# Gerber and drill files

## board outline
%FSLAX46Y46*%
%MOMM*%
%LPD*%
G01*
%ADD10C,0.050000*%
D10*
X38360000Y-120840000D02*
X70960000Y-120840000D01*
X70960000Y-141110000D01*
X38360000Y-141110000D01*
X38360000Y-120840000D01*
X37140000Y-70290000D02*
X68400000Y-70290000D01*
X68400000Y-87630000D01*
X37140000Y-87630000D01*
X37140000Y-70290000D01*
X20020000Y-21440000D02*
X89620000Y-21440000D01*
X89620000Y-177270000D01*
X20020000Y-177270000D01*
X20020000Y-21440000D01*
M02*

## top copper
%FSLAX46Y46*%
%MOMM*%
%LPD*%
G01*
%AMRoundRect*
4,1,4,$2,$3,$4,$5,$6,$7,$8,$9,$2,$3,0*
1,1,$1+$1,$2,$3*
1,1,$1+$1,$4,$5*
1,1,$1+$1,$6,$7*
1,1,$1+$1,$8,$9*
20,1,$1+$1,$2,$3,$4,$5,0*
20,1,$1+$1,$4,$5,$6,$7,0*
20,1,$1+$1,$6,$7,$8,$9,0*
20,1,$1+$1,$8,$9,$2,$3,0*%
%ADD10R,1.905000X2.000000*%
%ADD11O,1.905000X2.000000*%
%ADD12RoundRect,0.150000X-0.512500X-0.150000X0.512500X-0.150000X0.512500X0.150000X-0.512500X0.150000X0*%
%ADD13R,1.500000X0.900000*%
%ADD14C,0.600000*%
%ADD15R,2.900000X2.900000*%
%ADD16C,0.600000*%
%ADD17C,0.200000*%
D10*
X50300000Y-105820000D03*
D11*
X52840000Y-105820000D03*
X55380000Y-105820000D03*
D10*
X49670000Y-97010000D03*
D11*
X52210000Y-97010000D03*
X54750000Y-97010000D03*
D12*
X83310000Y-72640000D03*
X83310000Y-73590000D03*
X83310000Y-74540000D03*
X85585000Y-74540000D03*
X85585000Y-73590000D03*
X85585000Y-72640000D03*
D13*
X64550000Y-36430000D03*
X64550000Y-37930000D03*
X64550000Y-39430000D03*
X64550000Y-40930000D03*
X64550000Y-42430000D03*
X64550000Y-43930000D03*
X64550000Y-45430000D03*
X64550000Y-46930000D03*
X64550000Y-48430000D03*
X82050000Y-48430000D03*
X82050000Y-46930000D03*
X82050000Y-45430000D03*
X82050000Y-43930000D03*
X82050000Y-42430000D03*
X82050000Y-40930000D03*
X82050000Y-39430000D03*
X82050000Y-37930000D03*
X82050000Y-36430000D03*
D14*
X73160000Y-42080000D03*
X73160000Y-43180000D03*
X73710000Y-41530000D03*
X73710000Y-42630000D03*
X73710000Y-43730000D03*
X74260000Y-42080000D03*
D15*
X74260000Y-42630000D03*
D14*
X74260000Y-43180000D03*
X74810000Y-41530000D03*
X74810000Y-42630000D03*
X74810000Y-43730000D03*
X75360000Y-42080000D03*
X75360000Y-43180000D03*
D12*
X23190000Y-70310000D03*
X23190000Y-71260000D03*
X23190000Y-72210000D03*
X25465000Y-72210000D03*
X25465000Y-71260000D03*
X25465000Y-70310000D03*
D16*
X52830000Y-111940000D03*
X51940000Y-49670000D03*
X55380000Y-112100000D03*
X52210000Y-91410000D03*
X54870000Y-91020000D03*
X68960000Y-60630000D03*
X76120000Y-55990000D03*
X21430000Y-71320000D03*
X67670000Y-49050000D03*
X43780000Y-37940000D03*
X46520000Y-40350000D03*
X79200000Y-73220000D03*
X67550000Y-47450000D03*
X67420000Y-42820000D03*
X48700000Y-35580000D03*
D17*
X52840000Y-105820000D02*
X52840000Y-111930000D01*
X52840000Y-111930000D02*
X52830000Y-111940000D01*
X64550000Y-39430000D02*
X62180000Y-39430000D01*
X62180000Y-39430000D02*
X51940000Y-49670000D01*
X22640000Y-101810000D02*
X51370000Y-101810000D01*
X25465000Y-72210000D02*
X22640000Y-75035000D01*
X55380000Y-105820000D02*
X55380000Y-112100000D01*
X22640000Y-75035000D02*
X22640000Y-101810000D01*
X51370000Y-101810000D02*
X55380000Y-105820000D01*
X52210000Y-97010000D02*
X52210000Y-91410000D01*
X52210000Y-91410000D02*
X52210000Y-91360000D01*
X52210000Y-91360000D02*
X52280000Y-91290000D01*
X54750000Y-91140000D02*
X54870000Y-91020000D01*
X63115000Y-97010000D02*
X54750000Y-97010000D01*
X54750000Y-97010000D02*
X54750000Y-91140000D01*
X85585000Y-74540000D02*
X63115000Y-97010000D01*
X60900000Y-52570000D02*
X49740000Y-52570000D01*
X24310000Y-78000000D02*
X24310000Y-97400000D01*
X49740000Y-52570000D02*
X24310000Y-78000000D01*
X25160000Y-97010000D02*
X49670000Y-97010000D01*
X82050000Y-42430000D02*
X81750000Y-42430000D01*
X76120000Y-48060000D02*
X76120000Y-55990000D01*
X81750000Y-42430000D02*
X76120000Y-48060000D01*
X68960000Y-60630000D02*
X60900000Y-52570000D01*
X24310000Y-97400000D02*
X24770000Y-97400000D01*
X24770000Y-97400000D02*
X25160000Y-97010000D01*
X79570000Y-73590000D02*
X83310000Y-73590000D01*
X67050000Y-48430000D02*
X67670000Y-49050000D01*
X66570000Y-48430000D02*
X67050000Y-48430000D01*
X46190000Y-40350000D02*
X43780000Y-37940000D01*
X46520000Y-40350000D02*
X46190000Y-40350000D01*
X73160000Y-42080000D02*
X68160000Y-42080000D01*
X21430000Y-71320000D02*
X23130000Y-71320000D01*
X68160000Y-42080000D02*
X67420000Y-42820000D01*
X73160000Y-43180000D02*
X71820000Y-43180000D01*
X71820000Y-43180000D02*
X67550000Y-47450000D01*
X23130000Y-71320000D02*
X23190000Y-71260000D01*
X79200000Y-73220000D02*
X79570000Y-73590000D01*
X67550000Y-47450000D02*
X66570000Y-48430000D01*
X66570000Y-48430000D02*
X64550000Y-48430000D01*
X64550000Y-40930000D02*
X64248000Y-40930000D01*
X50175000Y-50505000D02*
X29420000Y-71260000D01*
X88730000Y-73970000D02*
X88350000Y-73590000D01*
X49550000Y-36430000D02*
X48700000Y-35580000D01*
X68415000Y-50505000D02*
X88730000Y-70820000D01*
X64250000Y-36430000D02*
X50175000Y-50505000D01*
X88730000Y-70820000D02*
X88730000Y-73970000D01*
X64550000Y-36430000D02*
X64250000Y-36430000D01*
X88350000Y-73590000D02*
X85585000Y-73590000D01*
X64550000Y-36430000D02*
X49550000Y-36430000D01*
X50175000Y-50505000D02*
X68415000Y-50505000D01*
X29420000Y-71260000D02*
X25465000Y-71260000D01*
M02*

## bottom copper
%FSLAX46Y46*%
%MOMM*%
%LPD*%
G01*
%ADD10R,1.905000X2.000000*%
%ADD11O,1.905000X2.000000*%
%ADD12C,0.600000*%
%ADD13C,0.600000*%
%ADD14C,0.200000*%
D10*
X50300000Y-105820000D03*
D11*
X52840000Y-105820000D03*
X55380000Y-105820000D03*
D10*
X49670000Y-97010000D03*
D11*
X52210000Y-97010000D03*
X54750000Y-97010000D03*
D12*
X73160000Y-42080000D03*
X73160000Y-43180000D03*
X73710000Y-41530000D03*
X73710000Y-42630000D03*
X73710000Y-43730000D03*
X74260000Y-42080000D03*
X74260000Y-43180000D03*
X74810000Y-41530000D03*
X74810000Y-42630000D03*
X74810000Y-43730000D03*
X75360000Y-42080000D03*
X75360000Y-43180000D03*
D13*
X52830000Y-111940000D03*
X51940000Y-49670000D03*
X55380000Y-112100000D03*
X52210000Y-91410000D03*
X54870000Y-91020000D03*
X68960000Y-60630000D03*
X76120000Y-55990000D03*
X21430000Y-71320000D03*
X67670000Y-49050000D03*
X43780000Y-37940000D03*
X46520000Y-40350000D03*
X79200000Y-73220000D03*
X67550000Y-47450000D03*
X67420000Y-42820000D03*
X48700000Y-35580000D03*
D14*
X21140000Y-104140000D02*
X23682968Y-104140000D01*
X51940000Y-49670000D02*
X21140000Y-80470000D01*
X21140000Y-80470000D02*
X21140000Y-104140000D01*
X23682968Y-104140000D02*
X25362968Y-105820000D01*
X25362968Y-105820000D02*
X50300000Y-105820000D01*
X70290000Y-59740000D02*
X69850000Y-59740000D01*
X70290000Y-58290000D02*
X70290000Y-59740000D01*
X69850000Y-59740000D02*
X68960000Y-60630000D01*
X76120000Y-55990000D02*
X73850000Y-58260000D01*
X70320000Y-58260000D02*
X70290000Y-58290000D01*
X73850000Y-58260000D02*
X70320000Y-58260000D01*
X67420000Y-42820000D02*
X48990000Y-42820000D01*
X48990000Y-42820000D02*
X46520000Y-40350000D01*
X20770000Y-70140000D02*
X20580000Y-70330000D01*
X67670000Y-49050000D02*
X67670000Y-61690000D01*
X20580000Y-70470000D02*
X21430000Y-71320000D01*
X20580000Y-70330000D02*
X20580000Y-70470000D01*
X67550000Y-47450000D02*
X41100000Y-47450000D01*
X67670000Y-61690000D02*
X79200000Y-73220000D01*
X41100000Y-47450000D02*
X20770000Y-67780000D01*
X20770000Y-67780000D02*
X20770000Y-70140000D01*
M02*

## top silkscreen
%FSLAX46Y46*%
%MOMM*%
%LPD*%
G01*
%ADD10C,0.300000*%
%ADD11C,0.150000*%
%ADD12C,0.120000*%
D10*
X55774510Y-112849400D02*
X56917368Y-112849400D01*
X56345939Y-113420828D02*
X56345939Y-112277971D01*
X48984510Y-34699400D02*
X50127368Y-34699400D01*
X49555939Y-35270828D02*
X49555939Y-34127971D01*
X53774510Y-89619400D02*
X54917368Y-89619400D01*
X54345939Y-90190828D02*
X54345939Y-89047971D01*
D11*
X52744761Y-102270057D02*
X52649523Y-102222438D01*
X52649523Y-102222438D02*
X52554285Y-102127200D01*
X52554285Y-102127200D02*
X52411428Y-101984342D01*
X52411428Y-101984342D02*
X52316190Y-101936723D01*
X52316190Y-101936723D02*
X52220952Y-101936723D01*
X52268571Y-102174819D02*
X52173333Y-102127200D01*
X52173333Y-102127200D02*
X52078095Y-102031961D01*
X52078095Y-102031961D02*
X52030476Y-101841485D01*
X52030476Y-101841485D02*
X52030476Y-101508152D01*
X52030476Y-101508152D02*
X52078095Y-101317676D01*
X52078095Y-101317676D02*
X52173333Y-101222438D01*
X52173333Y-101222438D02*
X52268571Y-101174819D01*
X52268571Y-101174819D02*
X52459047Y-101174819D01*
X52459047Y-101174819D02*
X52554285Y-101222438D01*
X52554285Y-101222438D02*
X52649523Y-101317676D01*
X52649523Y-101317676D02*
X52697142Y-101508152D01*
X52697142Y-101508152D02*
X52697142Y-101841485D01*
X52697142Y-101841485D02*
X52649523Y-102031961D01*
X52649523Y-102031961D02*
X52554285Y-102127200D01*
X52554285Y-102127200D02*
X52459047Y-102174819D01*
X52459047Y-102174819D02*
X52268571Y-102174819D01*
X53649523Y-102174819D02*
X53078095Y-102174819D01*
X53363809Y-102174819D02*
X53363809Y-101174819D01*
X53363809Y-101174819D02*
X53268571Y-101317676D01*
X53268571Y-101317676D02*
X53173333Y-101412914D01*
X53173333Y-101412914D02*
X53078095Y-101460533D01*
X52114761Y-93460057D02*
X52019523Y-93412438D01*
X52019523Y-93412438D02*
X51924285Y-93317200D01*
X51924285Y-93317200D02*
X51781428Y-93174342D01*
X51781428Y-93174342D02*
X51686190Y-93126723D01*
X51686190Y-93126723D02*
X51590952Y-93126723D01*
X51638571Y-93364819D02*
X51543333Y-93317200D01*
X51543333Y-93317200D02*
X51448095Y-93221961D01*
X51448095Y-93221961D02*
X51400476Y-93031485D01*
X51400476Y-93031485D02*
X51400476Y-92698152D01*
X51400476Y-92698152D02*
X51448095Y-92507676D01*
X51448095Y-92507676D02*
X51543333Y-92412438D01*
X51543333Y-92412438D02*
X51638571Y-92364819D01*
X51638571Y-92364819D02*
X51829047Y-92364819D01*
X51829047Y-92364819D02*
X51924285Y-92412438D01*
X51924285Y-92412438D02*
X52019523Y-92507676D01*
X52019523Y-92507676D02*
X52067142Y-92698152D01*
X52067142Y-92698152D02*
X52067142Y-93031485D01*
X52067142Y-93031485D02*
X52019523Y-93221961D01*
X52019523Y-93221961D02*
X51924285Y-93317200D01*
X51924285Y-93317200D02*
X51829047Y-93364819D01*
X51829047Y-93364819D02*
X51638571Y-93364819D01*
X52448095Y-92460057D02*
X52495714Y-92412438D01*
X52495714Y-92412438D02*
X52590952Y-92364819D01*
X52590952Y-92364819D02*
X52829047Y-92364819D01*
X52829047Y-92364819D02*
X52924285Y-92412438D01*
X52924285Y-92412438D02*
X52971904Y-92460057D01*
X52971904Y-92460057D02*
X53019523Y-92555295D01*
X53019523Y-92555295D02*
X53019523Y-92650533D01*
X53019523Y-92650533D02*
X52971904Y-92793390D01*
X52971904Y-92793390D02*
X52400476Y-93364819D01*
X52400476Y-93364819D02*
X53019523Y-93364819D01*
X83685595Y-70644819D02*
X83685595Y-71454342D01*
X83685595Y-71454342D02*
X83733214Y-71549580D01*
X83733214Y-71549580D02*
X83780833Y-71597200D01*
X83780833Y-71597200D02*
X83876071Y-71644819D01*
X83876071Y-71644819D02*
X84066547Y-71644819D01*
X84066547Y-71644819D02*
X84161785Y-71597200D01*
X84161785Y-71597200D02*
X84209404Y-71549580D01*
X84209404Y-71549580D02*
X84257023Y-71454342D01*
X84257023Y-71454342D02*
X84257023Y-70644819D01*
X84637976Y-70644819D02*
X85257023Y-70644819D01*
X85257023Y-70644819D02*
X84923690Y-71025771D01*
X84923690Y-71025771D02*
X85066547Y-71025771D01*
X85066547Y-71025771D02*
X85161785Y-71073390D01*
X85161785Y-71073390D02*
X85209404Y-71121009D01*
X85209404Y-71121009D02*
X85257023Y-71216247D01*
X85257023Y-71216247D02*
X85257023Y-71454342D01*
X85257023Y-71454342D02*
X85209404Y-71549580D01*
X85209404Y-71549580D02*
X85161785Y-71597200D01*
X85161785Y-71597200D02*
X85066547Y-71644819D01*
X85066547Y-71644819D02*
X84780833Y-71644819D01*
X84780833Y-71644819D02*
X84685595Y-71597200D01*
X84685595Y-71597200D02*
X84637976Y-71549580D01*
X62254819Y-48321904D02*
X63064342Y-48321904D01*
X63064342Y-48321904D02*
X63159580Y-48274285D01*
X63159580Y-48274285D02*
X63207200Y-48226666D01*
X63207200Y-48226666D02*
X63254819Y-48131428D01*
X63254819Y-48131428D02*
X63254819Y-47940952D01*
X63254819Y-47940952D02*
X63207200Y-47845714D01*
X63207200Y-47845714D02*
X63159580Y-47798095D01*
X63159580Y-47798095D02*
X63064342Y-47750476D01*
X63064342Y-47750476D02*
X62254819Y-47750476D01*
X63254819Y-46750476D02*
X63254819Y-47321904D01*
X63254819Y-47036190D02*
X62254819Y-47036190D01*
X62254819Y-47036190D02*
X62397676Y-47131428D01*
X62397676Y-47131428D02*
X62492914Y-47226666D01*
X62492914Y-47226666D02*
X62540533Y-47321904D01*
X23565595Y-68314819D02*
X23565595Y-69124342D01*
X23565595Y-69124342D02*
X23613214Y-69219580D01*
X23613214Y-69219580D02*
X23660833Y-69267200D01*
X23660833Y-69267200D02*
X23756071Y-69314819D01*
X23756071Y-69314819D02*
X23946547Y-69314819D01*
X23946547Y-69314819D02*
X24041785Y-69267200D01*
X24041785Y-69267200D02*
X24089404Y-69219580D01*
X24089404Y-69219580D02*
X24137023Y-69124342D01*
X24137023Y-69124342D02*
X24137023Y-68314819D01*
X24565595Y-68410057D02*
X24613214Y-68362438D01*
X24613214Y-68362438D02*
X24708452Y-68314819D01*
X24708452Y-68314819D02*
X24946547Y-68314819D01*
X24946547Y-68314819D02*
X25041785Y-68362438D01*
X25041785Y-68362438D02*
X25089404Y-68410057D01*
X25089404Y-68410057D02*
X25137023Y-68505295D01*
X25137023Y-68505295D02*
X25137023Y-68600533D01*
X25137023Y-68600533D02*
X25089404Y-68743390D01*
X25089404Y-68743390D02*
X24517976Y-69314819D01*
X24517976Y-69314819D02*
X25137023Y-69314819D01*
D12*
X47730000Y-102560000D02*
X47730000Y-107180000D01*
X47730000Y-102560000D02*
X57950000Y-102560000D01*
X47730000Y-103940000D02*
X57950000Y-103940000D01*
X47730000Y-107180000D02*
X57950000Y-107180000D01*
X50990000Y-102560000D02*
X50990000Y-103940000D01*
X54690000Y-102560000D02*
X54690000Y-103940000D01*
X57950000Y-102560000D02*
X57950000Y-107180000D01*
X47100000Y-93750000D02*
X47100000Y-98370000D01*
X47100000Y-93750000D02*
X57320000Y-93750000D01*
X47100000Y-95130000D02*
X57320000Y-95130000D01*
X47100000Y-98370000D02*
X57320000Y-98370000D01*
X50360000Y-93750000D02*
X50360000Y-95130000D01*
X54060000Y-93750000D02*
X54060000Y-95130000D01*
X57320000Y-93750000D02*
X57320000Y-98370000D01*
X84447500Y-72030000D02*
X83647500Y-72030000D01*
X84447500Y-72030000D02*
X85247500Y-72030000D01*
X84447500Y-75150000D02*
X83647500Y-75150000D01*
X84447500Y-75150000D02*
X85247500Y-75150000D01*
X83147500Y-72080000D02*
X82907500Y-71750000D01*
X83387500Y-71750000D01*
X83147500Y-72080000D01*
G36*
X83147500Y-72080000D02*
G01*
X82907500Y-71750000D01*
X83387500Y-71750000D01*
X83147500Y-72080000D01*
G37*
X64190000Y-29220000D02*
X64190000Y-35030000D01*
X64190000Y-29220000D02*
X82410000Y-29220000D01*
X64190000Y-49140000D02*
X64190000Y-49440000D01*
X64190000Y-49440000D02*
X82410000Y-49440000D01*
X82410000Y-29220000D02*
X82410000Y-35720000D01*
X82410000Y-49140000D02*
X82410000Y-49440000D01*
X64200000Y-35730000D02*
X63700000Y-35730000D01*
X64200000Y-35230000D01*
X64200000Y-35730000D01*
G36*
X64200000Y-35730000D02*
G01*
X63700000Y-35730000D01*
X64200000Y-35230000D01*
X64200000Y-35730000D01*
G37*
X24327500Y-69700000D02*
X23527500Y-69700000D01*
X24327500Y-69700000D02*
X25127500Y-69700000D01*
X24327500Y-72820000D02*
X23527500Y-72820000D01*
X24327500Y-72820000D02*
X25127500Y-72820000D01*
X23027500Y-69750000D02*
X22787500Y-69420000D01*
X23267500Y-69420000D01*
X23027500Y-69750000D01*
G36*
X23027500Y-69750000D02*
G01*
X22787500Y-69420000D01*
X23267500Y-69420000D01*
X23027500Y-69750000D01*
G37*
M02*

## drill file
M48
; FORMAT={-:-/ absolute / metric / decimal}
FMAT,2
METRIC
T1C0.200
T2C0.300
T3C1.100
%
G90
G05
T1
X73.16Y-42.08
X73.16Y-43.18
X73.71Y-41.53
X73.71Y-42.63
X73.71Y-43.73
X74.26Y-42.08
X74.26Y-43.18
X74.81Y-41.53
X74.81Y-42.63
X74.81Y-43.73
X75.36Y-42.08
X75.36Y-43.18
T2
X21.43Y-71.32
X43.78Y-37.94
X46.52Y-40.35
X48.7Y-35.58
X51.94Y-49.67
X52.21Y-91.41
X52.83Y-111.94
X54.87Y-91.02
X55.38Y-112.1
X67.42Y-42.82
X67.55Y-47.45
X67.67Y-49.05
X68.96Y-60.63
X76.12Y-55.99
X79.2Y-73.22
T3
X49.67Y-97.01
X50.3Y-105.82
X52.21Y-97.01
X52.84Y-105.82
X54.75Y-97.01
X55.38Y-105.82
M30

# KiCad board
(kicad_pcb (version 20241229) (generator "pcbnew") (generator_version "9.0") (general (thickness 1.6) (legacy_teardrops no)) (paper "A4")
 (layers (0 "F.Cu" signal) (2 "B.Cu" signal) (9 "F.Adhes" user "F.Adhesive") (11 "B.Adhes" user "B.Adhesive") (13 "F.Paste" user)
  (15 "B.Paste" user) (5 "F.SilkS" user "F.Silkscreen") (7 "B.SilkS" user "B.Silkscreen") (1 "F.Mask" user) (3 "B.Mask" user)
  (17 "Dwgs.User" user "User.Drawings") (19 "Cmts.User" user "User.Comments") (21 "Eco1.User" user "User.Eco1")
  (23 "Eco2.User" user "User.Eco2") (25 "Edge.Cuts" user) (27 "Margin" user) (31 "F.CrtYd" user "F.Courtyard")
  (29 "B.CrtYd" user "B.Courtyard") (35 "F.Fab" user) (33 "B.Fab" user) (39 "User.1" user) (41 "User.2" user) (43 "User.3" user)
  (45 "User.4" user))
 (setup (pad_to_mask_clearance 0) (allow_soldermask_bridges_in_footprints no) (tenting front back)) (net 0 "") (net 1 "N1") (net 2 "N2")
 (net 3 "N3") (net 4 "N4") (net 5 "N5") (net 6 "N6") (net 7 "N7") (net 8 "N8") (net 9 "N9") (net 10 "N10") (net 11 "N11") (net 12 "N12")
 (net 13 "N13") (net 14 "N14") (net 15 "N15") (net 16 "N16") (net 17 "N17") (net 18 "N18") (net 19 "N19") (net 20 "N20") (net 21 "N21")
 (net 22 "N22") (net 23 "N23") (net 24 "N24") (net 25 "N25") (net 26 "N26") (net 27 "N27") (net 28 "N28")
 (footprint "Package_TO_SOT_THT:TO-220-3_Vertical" (layer "F.Cu") (at 50.3 105.82)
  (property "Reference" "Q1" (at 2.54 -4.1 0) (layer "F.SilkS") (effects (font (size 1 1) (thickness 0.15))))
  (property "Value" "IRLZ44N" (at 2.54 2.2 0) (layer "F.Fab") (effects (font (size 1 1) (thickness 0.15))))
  (fp_line (start -2.57 -3.26) (end -2.57 1.36) (stroke (width 0.12) (type solid)) (layer "F.SilkS"))
  (fp_line (start -2.57 -3.26) (end 7.65 -3.26) (stroke (width 0.12) (type solid)) (layer "F.SilkS"))
  (fp_line (start -2.57 -1.88) (end 7.65 -1.88) (stroke (width 0.12) (type solid)) (layer "F.SilkS"))
  (fp_line (start -2.57 1.36) (end 7.65 1.36) (stroke (width 0.12) (type solid)) (layer "F.SilkS"))
  (fp_line (start 0.69 -3.26) (end 0.69 -1.88) (stroke (width 0.12) (type solid)) (layer "F.SilkS"))
  (fp_line (start 4.39 -3.26) (end 4.39 -1.88) (stroke (width 0.12) (type solid)) (layer "F.SilkS"))
  (fp_line (start 7.65 -3.26) (end 7.65 1.36) (stroke (width 0.12) (type solid)) (layer "F.SilkS"))
  (pad "1" thru_hole rect (at 0 0) (size 1.905 2) (drill 1.1) (layers "*.Cu" "*.Mask") (remove_unused_layers no) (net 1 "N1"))
  (pad "2" thru_hole oval (at 2.54 0) (size 1.905 2) (drill 1.1) (layers "*.Cu" "*.Mask") (remove_unused_layers no) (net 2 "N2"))
  (pad "3" thru_hole oval (at 5.08 0) (size 1.905 2) (drill 1.1) (layers "*.Cu" "*.Mask") (remove_unused_layers no) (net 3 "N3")))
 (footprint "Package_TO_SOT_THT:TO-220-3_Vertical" (layer "F.Cu") (at 49.67 97.01)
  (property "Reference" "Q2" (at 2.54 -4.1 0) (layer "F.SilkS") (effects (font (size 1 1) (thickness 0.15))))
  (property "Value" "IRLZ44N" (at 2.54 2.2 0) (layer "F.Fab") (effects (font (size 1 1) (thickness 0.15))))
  (fp_line (start -2.57 -3.26) (end -2.57 1.36) (stroke (width 0.12) (type solid)) (layer "F.SilkS"))
  (fp_line (start -2.57 -3.26) (end 7.65 -3.26) (stroke (width 0.12) (type solid)) (layer "F.SilkS"))
  (fp_line (start -2.57 -1.88) (end 7.65 -1.88) (stroke (width 0.12) (type solid)) (layer "F.SilkS"))
  (fp_line (start -2.57 1.36) (end 7.65 1.36) (stroke (width 0.12) (type solid)) (layer "F.SilkS"))
  (fp_line (start 0.69 -3.26) (end 0.69 -1.88) (stroke (width 0.12) (type solid)) (layer "F.SilkS"))
  (fp_line (start 4.39 -3.26) (end 4.39 -1.88) (stroke (width 0.12) (type solid)) (layer "F.SilkS"))
  (fp_line (start 7.65 -3.26) (end 7.65 1.36) (stroke (width 0.12) (type solid)) (layer "F.SilkS"))
  (pad "1" thru_hole rect (at 0 0) (size 1.905 2) (drill 1.1) (layers "*.Cu" "*.Mask") (remove_unused_layers no) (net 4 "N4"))
  (pad "2" thru_hole oval (at 2.54 0) (size 1.905 2) (drill 1.1) (layers "*.Cu" "*.Mask") (remove_unused_layers no) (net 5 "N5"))
  (pad "3" thru_hole oval (at 5.08 0) (size 1.905 2) (drill 1.1) (layers "*.Cu" "*.Mask") (remove_unused_layers no) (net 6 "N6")))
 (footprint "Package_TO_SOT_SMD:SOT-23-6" (layer "F.Cu") (at 84.4475 73.59)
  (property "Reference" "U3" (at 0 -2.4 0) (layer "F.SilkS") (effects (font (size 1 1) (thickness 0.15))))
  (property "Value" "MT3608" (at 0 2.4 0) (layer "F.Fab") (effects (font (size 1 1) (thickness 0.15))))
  (fp_line (start 0 -1.56) (end -0.8 -1.56) (stroke (width 0.12) (type solid)) (layer "F.SilkS"))
  (fp_line (start 0 -1.56) (end 0.8 -1.56) (stroke (width 0.12) (type solid)) (layer "F.SilkS"))
  (fp_line (start 0 1.56) (end -0.8 1.56) (stroke (width 0.12) (type solid)) (layer "F.SilkS"))
  (fp_line (start 0 1.56) (end 0.8 1.56) (stroke (width 0.12) (type solid)) (layer "F.SilkS"))
  (fp_poly (pts (xy -1.3 -1.51) (xy -1.54 -1.84) (xy -1.06 -1.84)) (stroke (width 0.12) (type solid)) (fill yes) (layer "F.SilkS"))
  (pad "1" smd roundrect (at -1.1375 -0.95) (size 1.325 0.6) (layers "F.Cu" "F.Mask" "F.Paste") (roundrect_rratio 0.25) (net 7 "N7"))
  (pad "2" smd roundrect (at -1.1375 0) (size 1.325 0.6) (layers "F.Cu" "F.Mask" "F.Paste") (roundrect_rratio 0.25) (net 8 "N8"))
  (pad "3" smd roundrect (at -1.1375 0.95) (size 1.325 0.6) (layers "F.Cu" "F.Mask" "F.Paste") (roundrect_rratio 0.25) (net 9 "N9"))
  (pad "4" smd roundrect (at 1.1375 0.95) (size 1.325 0.6) (layers "F.Cu" "F.Mask" "F.Paste") (roundrect_rratio 0.25) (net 6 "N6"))
  (pad "5" smd roundrect (at 1.1375 0) (size 1.325 0.6) (layers "F.Cu" "F.Mask" "F.Paste") (roundrect_rratio 0.25) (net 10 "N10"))
  (pad "6" smd roundrect (at 1.1375 -0.95) (size 1.325 0.6) (layers "F.Cu" "F.Mask" "F.Paste") (roundrect_rratio 0.25) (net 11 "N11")))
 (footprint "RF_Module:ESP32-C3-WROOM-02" (layer "F.Cu") (at 73.3 42.43)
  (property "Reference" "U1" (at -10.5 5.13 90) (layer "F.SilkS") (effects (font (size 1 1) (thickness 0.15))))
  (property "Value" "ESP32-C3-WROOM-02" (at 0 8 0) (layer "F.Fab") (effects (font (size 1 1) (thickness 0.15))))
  (fp_line (start -9.11 -13.21) (end -9.11 -7.4) (stroke (width 0.12) (type solid)) (layer "F.SilkS"))
  (fp_line (start -9.11 -13.21) (end 9.11 -13.21) (stroke (width 0.12) (type solid)) (layer "F.SilkS"))
  (fp_line (start -9.11 6.71) (end -9.11 7.01) (stroke (width 0.12) (type solid)) (layer "F.SilkS"))
  (fp_line (start -9.11 7.01) (end 9.11 7.01) (stroke (width 0.12) (type solid)) (layer "F.SilkS"))
  (fp_line (start 9.11 -13.21) (end 9.11 -6.71) (stroke (width 0.12) (type solid)) (layer "F.SilkS"))
  (fp_line (start 9.11 6.71) (end 9.11 7.01) (stroke (width 0.12) (type solid)) (layer "F.SilkS"))
  (fp_poly
   (pts (xy -9.1 -6.7) (xy -9.6 -6.7) (xy -9.1 -7.2) (xy -9.1 -6.7)) (stroke (width 0.12) (type solid)) (fill yes) (layer "F.SilkS"))
  (pad "" smd rect (at -0.14 -0.9) (size 0.7 0.7) (layers "F.Paste"))
  (pad "" smd rect (at -0.14 0.2) (size 0.7 0.7) (layers "F.Paste"))
  (pad "" smd rect (at -0.14 1.3) (size 0.7 0.7) (layers "F.Paste"))
  (pad "" smd rect (at 0.96 -0.9) (size 0.7 0.7) (layers "F.Paste"))
  (pad "" smd rect (at 0.96 0.2) (size 0.7 0.7) (layers "F.Paste"))
  (pad "" smd rect (at 0.96 1.3) (size 0.7 0.7) (layers "F.Paste"))
  (pad "" smd rect (at 2.06 -0.9) (size 0.7 0.7) (layers "F.Paste"))
  (pad "" smd rect (at 2.06 0.2) (size 0.7 0.7) (layers "F.Paste"))
  (pad "" smd rect (at 2.06 1.3) (size 0.7 0.7) (layers "F.Paste"))
  (pad "1" smd rect (at -8.75 -6) (size 1.5 0.9) (layers "F.Cu" "F.Mask" "F.Paste") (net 10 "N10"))
  (pad "2" smd rect (at -8.75 -4.5) (size 1.5 0.9) (layers "F.Cu" "F.Mask" "F.Paste") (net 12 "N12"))
  (pad "3" smd rect (at -8.75 -3) (size 1.5 0.9) (layers "F.Cu" "F.Mask" "F.Paste") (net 1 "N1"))
  (pad "4" smd rect (at -8.75 -1.5) (size 1.5 0.9) (layers "F.Cu" "F.Mask" "F.Paste") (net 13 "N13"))
  (pad "5" smd rect (at -8.75 0) (size 1.5 0.9) (layers "F.Cu" "F.Mask" "F.Paste") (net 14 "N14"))
  (pad "6" smd rect (at -8.75 1.5) (size 1.5 0.9) (layers "F.Cu" "F.Mask" "F.Paste") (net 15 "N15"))
  (pad "7" smd rect (at -8.75 3) (size 1.5 0.9) (layers "F.Cu" "F.Mask" "F.Paste") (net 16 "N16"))
  (pad "8" smd rect (at -8.75 4.5) (size 1.5 0.9) (layers "F.Cu" "F.Mask" "F.Paste") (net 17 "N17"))
  (pad "9" smd rect (at -8.75 6) (size 1.5 0.9) (layers "F.Cu" "F.Mask" "F.Paste") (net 8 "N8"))
  (pad "10" smd rect (at 8.75 6) (size 1.5 0.9) (layers "F.Cu" "F.Mask" "F.Paste") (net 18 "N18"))
  (pad "11" smd rect (at 8.75 4.5) (size 1.5 0.9) (layers "F.Cu" "F.Mask" "F.Paste") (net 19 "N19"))
  (pad "12" smd rect (at 8.75 3) (size 1.5 0.9) (layers "F.Cu" "F.Mask" "F.Paste") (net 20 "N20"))
  (pad "13" smd rect (at 8.75 1.5) (size 1.5 0.9) (layers "F.Cu" "F.Mask" "F.Paste") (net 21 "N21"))
  (pad "14" smd rect (at 8.75 0) (size 1.5 0.9) (layers "F.Cu" "F.Mask" "F.Paste") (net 4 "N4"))
  (pad "15" smd rect (at 8.75 -1.5) (size 1.5 0.9) (layers "F.Cu" "F.Mask" "F.Paste") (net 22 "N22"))
  (pad "16" smd rect (at 8.75 -3) (size 1.5 0.9) (layers "F.Cu" "F.Mask" "F.Paste") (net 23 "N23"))
  (pad "17" smd rect (at 8.75 -4.5) (size 1.5 0.9) (layers "F.Cu" "F.Mask" "F.Paste") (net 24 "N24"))
  (pad "18" smd rect (at 8.75 -6) (size 1.5 0.9) (layers "F.Cu" "F.Mask" "F.Paste") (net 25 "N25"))
  (pad "19" thru_hole circle (at -0.14 -0.35) (size 0.6 0.6) (drill 0.2) (layers "*.Cu" "F.Mask") (remove_unused_layers no) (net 8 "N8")
   (zone_connect 2))
  (pad "19" thru_hole circle (at -0.14 0.75) (size 0.6 0.6) (drill 0.2) (layers "*.Cu" "F.Mask") (remove_unused_layers no) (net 8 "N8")
   (zone_connect 2))
  (pad "19" thru_hole circle (at 0.41 -0.9) (size 0.6 0.6) (drill 0.2) (layers "*.Cu" "F.Mask") (remove_unused_layers no) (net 8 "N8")
   (zone_connect 2))
  (pad "19" thru_hole circle (at 0.41 0.2) (size 0.6 0.6) (drill 0.2) (layers "*.Cu" "F.Mask") (remove_unused_layers no) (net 8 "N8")
   (zone_connect 2))
  (pad "19" thru_hole circle (at 0.41 1.3) (size 0.6 0.6) (drill 0.2) (layers "*.Cu" "F.Mask") (remove_unused_layers no) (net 8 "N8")
   (zone_connect 2))
  (pad "19" thru_hole circle (at 0.96 -0.35) (size 0.6 0.6) (drill 0.2) (layers "*.Cu" "F.Mask") (remove_unused_layers no) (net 8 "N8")
   (zone_connect 2))
  (pad "19" smd rect (at 0.96 0.2) (size 2.9 2.9) (layers "F.Cu" "F.Mask") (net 8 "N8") (zone_connect 2))
  (pad "19" thru_hole circle (at 0.96 0.75) (size 0.6 0.6) (drill 0.2) (layers "*.Cu" "F.Mask") (remove_unused_layers no) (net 8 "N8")
   (zone_connect 2))
  (pad "19" thru_hole circle (at 1.51 -0.9) (size 0.6 0.6) (drill 0.2) (layers "*.Cu" "F.Mask") (remove_unused_layers no) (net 8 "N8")
   (zone_connect 2))
  (pad "19" thru_hole circle (at 1.51 0.2) (size 0.6 0.6) (drill 0.2) (layers "*.Cu" "F.Mask") (remove_unused_layers no) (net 8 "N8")
   (zone_connect 2))
  (pad "19" thru_hole circle (at 1.51 1.3) (size 0.6 0.6) (drill 0.2) (layers "*.Cu" "F.Mask") (remove_unused_layers no) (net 8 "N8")
   (zone_connect 2))
  (pad "19" thru_hole circle (at 2.06 -0.35) (size 0.6 0.6) (drill 0.2) (layers "*.Cu" "F.Mask") (remove_unused_layers no) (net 8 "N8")
   (zone_connect 2))
  (pad "19" thru_hole circle (at 2.06 0.75) (size 0.6 0.6) (drill 0.2) (layers "*.Cu" "F.Mask") (remove_unused_layers no) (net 8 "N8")
   (zone_connect 2))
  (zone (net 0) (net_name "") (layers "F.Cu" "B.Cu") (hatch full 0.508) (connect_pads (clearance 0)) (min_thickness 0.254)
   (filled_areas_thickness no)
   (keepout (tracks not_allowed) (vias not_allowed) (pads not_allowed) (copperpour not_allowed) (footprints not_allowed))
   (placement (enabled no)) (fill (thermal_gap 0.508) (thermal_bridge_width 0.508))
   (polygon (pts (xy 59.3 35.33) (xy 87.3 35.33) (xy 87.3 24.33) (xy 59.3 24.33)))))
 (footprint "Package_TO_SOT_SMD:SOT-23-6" (layer "F.Cu") (at 24.3275 71.26)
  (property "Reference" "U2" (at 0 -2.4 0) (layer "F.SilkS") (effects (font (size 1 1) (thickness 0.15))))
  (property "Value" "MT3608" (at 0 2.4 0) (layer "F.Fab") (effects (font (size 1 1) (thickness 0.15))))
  (fp_line (start 0 -1.56) (end -0.8 -1.56) (stroke (width 0.12) (type solid)) (layer "F.SilkS"))
  (fp_line (start 0 -1.56) (end 0.8 -1.56) (stroke (width 0.12) (type solid)) (layer "F.SilkS"))
  (fp_line (start 0 1.56) (end -0.8 1.56) (stroke (width 0.12) (type solid)) (layer "F.SilkS"))
  (fp_line (start 0 1.56) (end 0.8 1.56) (stroke (width 0.12) (type solid)) (layer "F.SilkS"))
  (fp_poly (pts (xy -1.3 -1.51) (xy -1.54 -1.84) (xy -1.06 -1.84)) (stroke (width 0.12) (type solid)) (fill yes) (layer "F.SilkS"))
  (pad "1" smd roundrect (at -1.1375 -0.95) (size 1.325 0.6) (layers "F.Cu" "F.Mask" "F.Paste") (roundrect_rratio 0.25) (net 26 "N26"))
  (pad "2" smd roundrect (at -1.1375 0) (size 1.325 0.6) (layers "F.Cu" "F.Mask" "F.Paste") (roundrect_rratio 0.25) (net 8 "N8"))
  (pad "3" smd roundrect (at -1.1375 0.95) (size 1.325 0.6) (layers "F.Cu" "F.Mask" "F.Paste") (roundrect_rratio 0.25) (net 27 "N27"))
  (pad "4" smd roundrect (at 1.1375 0.95) (size 1.325 0.6) (layers "F.Cu" "F.Mask" "F.Paste") (roundrect_rratio 0.25) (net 3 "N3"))
  (pad "5" smd roundrect (at 1.1375 0) (size 1.325 0.6) (layers "F.Cu" "F.Mask" "F.Paste") (roundrect_rratio 0.25) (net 10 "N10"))
  (pad "6" smd roundrect (at 1.1375 -0.95) (size 1.325 0.6) (layers "F.Cu" "F.Mask" "F.Paste") (roundrect_rratio 0.25) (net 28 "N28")))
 (gr_rect (start 38.36 120.84) (end 70.96 141.11) (stroke (width 0.05) (type default)) (fill no) (layer "Edge.Cuts"))
 (gr_rect (start 37.14 70.29) (end 68.4 87.63) (stroke (width 0.05) (type default)) (fill no) (layer "Edge.Cuts"))
 (gr_rect (start 20.02 21.44) (end 89.62 177.27) (stroke (width 0.05) (type default)) (fill no) (layer "Edge.Cuts"))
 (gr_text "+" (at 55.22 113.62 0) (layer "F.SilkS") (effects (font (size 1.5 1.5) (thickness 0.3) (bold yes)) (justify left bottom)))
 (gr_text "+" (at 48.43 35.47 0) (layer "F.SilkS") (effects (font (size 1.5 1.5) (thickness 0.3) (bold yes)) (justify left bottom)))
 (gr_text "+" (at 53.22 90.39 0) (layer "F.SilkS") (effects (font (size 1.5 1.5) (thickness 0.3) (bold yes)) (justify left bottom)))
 (segment (start 52.84 105.82) (end 52.84 111.93) (width 0.2) (layer "F.Cu") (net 2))
 (segment (start 52.84 111.93) (end 52.83 111.94) (width 0.2) (layer "F.Cu") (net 2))
 (via (at 52.83 111.94) (size 0.6) (drill 0.3) (layers "F.Cu" "B.Cu") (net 2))
 (segment (start 64.55 39.43) (end 62.18 39.43) (width 0.2) (layer "F.Cu") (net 1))
 (segment (start 62.18 39.43) (end 51.94 49.67) (width 0.2) (layer "F.Cu") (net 1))
 (via (at 51.94 49.67) (size 0.6) (drill 0.3) (layers "F.Cu" "B.Cu") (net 1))
 (segment (start 21.14 104.14) (end 23.682968 104.14) (width 0.2) (layer "B.Cu") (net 1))
 (segment (start 51.94 49.67) (end 21.14 80.47) (width 0.2) (layer "B.Cu") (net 1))
 (segment (start 21.14 80.47) (end 21.14 104.14) (width 0.2) (layer "B.Cu") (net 1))
 (segment (start 23.682968 104.14) (end 25.362968 105.82) (width 0.2) (layer "B.Cu") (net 1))
 (segment (start 25.362968 105.82) (end 50.3 105.82) (width 0.2) (layer "B.Cu") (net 1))
 (segment (start 22.64 101.81) (end 51.37 101.81) (width 0.2) (layer "F.Cu") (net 3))
 (segment (start 25.465 72.21) (end 22.64 75.035) (width 0.2) (layer "F.Cu") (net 3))
 (segment (start 55.38 105.82) (end 55.38 112.1) (width 0.2) (layer "F.Cu") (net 3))
 (segment (start 22.64 75.035) (end 22.64 101.81) (width 0.2) (layer "F.Cu") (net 3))
 (segment (start 51.37 101.81) (end 55.38 105.82) (width 0.2) (layer "F.Cu") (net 3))
 (via (at 55.38 112.1) (size 0.6) (drill 0.3) (layers "F.Cu" "B.Cu") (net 3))
 (segment (start 52.21 97.01) (end 52.21 91.41) (width 0.2) (layer "F.Cu") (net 5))
 (segment (start 52.21 91.41) (end 52.21 91.36) (width 0.2) (layer "F.Cu") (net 5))
 (segment (start 52.21 91.36) (end 52.28 91.29) (width 0.2) (layer "F.Cu") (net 5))
 (via (at 52.21 91.41) (size 0.6) (drill 0.3) (layers "F.Cu" "B.Cu") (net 5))
 (segment (start 54.75 91.14) (end 54.87 91.02) (width 0.2) (layer "F.Cu") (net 6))
 (segment (start 63.115 97.01) (end 54.75 97.01) (width 0.2) (layer "F.Cu") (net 6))
 (segment (start 54.75 97.01) (end 54.75 91.14) (width 0.2) (layer "F.Cu") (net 6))
 (segment (start 85.585 74.54) (end 63.115 97.01) (width 0.2) (layer "F.Cu") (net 6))
 (via (at 54.87 91.02) (size 0.6) (drill 0.3) (layers "F.Cu" "B.Cu") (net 6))
 (segment (start 60.9 52.57) (end 49.74 52.57) (width 0.2) (layer "F.Cu") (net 4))
 (segment (start 24.31 78) (end 24.31 97.4) (width 0.2) (layer "F.Cu") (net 4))
 (segment (start 49.74 52.57) (end 24.31 78) (width 0.2) (layer "F.Cu") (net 4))
 (segment (start 25.16 97.01) (end 49.67 97.01) (width 0.2) (layer "F.Cu") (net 4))
 (segment (start 82.05 42.43) (end 81.75 42.43) (width 0.2) (layer "F.Cu") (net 4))
 (segment (start 76.12 48.06) (end 76.12 55.99) (width 0.2) (layer "F.Cu") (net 4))
 (segment (start 81.75 42.43) (end 76.12 48.06) (width 0.2) (layer "F.Cu") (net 4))
 (segment (start 68.96 60.63) (end 60.9 52.57) (width 0.2) (layer "F.Cu") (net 4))
 (segment (start 24.31 97.4) (end 24.77 97.4) (width 0.2) (layer "F.Cu") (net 4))
 (segment (start 24.77 97.4) (end 25.16 97.01) (width 0.2) (layer "F.Cu") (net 4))
 (via (at 68.96 60.63) (size 0.6) (drill 0.3) (layers "F.Cu" "B.Cu") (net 4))
 (via (at 76.12 55.99) (size 0.6) (drill 0.3) (layers "F.Cu" "B.Cu") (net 4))
 (segment (start 70.29 59.74) (end 69.85 59.74) (width 0.2) (layer "B.Cu") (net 4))
 (segment (start 70.29 58.29) (end 70.29 59.74) (width 0.2) (layer "B.Cu") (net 4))
 (segment (start 69.85 59.74) (end 68.96 60.63) (width 0.2) (layer "B.Cu") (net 4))
 (segment (start 76.12 55.99) (end 73.85 58.26) (width 0.2) (layer "B.Cu") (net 4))
 (segment (start 70.32 58.26) (end 70.29 58.29) (width 0.2) (layer "B.Cu") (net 4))
 (segment (start 73.85 58.26) (end 70.32 58.26) (width 0.2) (layer "B.Cu") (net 4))
 (segment (start 79.57 73.59) (end 83.31 73.59) (width 0.2) (layer "F.Cu") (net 8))
 (segment (start 67.05 48.43) (end 67.67 49.05) (width 0.2) (layer "F.Cu") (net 8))
 (segment (start 66.57 48.43) (end 67.05 48.43) (width 0.2) (layer "F.Cu") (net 8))
 (segment (start 46.19 40.35) (end 43.78 37.94) (width 0.2) (layer "F.Cu") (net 8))
 (segment (start 46.52 40.35) (end 46.19 40.35) (width 0.2) (layer "F.Cu") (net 8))
 (segment (start 73.16 42.08) (end 68.16 42.08) (width 0.2) (layer "F.Cu") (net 8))
 (segment (start 21.43 71.32) (end 23.13 71.32) (width 0.2) (layer "F.Cu") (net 8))
 (segment (start 68.16 42.08) (end 67.42 42.82) (width 0.2) (layer "F.Cu") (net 8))
 (segment (start 73.16 43.18) (end 71.82 43.18) (width 0.2) (layer "F.Cu") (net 8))
 (segment (start 71.82 43.18) (end 67.55 47.45) (width 0.2) (layer "F.Cu") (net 8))
 (segment (start 23.13 71.32) (end 23.19 71.26) (width 0.2) (layer "F.Cu") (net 8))
 (segment (start 79.2 73.22) (end 79.57 73.59) (width 0.2) (layer "F.Cu") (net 8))
 (segment (start 67.55 47.45) (end 66.57 48.43) (width 0.2) (layer "F.Cu") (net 8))
 (segment (start 66.57 48.43) (end 64.55 48.43) (width 0.2) (layer "F.Cu") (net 8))
 (via (at 21.43 71.32) (size 0.6) (drill 0.3) (layers "F.Cu" "B.Cu") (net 8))
 (via (at 67.67 49.05) (size 0.6) (drill 0.3) (layers "F.Cu" "B.Cu") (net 8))
 (via (at 43.78 37.94) (size 0.6) (drill 0.3) (layers "F.Cu" "B.Cu") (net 8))
 (via (at 46.52 40.35) (size 0.6) (drill 0.3) (layers "F.Cu" "B.Cu") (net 8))
 (via (at 79.2 73.22) (size 0.6) (drill 0.3) (layers "F.Cu" "B.Cu") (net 8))
 (via (at 67.55 47.45) (size 0.6) (drill 0.3) (layers "F.Cu" "B.Cu") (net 8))
 (via (at 67.42 42.82) (size 0.6) (drill 0.3) (layers "F.Cu" "B.Cu") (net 8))
 (segment (start 67.42 42.82) (end 48.99 42.82) (width 0.2) (layer "B.Cu") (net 8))
 (segment (start 48.99 42.82) (end 46.52 40.35) (width 0.2) (layer "B.Cu") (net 8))
 (segment (start 20.77 70.14) (end 20.58 70.33) (width 0.2) (layer "B.Cu") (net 8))
 (segment (start 67.67 49.05) (end 67.67 61.69) (width 0.2) (layer "B.Cu") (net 8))
 (segment (start 20.58 70.47) (end 21.43 71.32) (width 0.2) (layer "B.Cu") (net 8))
 (segment (start 20.58 70.33) (end 20.58 70.47) (width 0.2) (layer "B.Cu") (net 8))
 (segment (start 67.55 47.45) (end 41.1 47.45) (width 0.2) (layer "B.Cu") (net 8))
 (segment (start 67.67 61.69) (end 79.2 73.22) (width 0.2) (layer "B.Cu") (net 8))
 (segment (start 41.1 47.45) (end 20.77 67.78) (width 0.2) (layer "B.Cu") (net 8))
 (segment (start 20.77 67.78) (end 20.77 70.14) (width 0.2) (layer "B.Cu") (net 8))
 (segment (start 64.55 40.93) (end 64.248 40.93) (width 0.2) (layer "F.Cu") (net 13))
 (segment (start 50.175 50.505) (end 29.42 71.26) (width 0.2) (layer "F.Cu") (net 10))
 (segment (start 88.73 73.97) (end 88.35 73.59) (width 0.2) (layer "F.Cu") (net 10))
 (segment (start 49.55 36.43) (end 48.7 35.58) (width 0.2) (layer "F.Cu") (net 10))
 (segment (start 68.415 50.505) (end 88.73 70.82) (width 0.2) (layer "F.Cu") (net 10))
 (segment (start 64.25 36.43) (end 50.175 50.505) (width 0.2) (layer "F.Cu") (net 10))
 (segment (start 88.73 70.82) (end 88.73 73.97) (width 0.2) (layer "F.Cu") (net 10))
 (segment (start 64.55 36.43) (end 64.25 36.43) (width 0.2) (layer "F.Cu") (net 10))
 (segment (start 88.35 73.59) (end 85.585 73.59) (width 0.2) (layer "F.Cu") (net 10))
 (segment (start 64.55 36.43) (end 49.55 36.43) (width 0.2) (layer "F.Cu") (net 10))
 (segment (start 50.175 50.505) (end 68.415 50.505) (width 0.2) (layer "F.Cu") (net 10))
 (segment (start 29.42 71.26) (end 25.465 71.26) (width 0.2) (layer "F.Cu") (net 10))
 (via (at 48.7 35.58) (size 0.6) (drill 0.3) (layers "F.Cu" "B.Cu") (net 10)))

